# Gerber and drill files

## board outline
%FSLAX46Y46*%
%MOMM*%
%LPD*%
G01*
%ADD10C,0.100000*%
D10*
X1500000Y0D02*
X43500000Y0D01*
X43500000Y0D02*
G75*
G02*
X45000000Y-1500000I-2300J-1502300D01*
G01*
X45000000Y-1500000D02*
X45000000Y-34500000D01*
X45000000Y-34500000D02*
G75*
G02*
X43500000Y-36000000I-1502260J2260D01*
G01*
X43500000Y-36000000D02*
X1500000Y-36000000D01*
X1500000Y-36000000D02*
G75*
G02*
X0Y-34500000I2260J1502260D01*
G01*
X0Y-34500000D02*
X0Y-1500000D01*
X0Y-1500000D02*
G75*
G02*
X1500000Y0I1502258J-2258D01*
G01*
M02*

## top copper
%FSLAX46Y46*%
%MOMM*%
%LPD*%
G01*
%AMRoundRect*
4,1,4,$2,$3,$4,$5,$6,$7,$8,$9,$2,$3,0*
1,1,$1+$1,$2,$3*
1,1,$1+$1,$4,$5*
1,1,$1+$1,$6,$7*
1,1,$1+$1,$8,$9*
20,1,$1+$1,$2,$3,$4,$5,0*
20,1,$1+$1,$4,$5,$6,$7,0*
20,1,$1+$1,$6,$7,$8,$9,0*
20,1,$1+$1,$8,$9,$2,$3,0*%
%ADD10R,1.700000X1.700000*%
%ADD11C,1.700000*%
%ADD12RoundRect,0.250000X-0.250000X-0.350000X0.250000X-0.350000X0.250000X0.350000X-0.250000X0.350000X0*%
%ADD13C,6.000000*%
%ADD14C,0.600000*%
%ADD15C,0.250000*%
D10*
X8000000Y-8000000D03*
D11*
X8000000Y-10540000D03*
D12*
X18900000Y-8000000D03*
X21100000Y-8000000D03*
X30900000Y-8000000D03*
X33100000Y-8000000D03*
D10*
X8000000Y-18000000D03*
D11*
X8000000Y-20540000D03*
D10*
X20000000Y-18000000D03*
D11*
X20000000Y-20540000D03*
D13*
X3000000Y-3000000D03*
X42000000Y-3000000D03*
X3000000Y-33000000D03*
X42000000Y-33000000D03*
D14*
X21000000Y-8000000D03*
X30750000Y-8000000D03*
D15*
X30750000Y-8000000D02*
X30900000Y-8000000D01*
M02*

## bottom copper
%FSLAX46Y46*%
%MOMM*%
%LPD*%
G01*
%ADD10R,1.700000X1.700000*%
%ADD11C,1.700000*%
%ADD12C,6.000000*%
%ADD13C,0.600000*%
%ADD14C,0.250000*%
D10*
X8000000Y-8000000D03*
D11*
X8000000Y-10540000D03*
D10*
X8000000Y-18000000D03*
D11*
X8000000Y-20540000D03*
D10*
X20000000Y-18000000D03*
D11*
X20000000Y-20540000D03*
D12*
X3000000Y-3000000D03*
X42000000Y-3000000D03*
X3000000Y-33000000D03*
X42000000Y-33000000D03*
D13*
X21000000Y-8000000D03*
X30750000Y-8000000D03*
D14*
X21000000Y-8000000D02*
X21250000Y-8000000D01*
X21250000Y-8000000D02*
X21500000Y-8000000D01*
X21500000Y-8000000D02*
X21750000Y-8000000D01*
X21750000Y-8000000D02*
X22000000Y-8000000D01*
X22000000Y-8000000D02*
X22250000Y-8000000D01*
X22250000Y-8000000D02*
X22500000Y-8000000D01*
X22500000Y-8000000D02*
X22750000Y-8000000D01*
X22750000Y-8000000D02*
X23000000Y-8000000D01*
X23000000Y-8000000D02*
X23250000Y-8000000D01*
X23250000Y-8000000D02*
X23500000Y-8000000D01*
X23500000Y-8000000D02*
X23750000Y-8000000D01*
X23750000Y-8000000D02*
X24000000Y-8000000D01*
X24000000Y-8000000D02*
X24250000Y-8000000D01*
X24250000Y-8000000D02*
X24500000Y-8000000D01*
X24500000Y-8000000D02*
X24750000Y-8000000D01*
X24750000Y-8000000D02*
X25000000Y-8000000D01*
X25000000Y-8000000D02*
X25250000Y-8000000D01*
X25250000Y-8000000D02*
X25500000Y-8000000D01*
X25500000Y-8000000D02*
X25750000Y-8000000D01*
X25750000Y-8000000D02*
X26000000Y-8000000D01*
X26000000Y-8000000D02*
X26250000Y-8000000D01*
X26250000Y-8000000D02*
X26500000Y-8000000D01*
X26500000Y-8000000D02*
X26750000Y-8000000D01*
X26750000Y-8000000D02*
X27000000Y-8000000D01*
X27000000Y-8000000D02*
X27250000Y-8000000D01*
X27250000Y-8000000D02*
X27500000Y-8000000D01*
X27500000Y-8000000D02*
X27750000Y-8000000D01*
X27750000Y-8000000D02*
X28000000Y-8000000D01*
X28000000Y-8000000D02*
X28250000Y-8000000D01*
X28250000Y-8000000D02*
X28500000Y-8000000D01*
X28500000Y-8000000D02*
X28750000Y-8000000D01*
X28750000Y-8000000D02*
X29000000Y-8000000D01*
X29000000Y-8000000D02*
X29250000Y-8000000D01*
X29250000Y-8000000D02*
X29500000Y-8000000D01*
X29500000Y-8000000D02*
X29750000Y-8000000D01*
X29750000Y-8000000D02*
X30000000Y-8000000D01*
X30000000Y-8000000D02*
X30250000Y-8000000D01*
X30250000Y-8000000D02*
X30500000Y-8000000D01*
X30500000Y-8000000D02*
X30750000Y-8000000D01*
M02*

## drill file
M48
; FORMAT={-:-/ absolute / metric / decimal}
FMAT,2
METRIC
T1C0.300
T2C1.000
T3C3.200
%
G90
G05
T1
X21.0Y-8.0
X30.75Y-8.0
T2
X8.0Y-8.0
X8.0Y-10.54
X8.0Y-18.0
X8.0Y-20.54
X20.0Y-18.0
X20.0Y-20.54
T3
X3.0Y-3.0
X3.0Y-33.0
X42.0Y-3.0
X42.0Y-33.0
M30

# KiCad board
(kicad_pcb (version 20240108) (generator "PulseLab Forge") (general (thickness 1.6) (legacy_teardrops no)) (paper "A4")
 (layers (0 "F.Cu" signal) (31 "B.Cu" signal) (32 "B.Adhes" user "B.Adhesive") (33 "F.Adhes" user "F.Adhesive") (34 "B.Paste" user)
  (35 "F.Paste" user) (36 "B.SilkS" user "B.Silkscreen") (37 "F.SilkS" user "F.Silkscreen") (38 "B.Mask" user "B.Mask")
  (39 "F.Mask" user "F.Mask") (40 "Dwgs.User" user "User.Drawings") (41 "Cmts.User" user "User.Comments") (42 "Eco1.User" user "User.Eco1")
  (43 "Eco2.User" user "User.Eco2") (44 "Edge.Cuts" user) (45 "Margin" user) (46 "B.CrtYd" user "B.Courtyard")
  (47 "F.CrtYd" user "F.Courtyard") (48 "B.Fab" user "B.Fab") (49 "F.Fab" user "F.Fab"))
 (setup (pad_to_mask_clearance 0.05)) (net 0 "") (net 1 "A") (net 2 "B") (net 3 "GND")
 (gr_line (start 1.500 0.000) (end 43.500 0.000) (layer "Edge.Cuts") (stroke (width 0.1)))
 (gr_arc (start 43.500 0.000) (mid 44.560 0.440) (end 45.000 1.500) (layer "Edge.Cuts") (stroke (width 0.1)))
 (gr_line (start 45.000 1.500) (end 45.000 34.500) (layer "Edge.Cuts") (stroke (width 0.1)))
 (gr_arc (start 45.000 34.500) (mid 44.560 35.560) (end 43.500 36.000) (layer "Edge.Cuts") (stroke (width 0.1)))
 (gr_line (start 43.500 36.000) (end 1.500 36.000) (layer "Edge.Cuts") (stroke (width 0.1)))
 (gr_arc (start 1.500 36.000) (mid 0.440 35.560) (end 0.000 34.500) (layer "Edge.Cuts") (stroke (width 0.1)))
 (gr_line (start 0.000 34.500) (end 0.000 1.500) (layer "Edge.Cuts") (stroke (width 0.1)))
 (gr_arc (start 0.000 1.500) (mid 0.440 0.440) (end 1.500 0.000) (layer "Edge.Cuts") (stroke (width 0.1)))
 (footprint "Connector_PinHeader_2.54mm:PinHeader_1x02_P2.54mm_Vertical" (layer "F.Cu") (at 8.0000 8.0000)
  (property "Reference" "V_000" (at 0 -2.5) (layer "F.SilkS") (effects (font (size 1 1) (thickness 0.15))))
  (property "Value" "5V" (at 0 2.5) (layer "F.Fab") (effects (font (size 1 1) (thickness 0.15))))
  (pad "1" thru_hole rect (at 0.0000 0.0000) (size 1.7000 1.7000) (drill 1.0) (layers "*.Cu" "*.Mask") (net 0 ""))
  (pad "2" thru_hole circle (at 0.0000 2.5400) (size 1.7000 1.7000) (drill 1.0) (layers "*.Cu" "*.Mask") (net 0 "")))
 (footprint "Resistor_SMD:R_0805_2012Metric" (layer "F.Cu") (at 20.0000 8.0000)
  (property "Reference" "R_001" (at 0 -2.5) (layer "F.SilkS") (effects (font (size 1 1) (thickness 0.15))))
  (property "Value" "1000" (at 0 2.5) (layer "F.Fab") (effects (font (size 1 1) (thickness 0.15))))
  (pad "1" smd roundrect (at -1.1000 0.0000) (size 1.0000 1.2000) (layers "F.Cu" "F.Paste" "F.Mask") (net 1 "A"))
  (pad "2" smd roundrect (at 1.1000 0.0000) (size 1.0000 1.2000) (layers "F.Cu" "F.Paste" "F.Mask") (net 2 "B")))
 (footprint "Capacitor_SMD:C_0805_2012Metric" (layer "F.Cu") (at 32.0000 8.0000)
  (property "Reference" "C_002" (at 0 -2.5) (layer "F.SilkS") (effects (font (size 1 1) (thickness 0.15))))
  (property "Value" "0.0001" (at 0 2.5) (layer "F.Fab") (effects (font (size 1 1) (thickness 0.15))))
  (pad "1" smd roundrect (at -1.1000 0.0000) (size 1.0000 1.2000) (layers "F.Cu" "F.Paste" "F.Mask") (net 2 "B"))
  (pad "2" smd roundrect (at 1.1000 0.0000) (size 1.0000 1.2000) (layers "F.Cu" "F.Paste" "F.Mask") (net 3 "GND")))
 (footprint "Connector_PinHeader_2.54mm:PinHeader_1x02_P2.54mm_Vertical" (layer "F.Cu") (at 8.0000 18.0000)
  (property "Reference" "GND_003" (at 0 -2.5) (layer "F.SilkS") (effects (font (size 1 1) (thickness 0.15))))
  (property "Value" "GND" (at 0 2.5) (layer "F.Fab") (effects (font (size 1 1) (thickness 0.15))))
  (pad "1" thru_hole rect (at 0.0000 0.0000) (size 1.7000 1.7000) (drill 1.0) (layers "*.Cu" "*.Mask") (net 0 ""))
  (pad "2" thru_hole circle (at 0.0000 2.5400) (size 1.7000 1.7000) (drill 1.0) (layers "*.Cu" "*.Mask") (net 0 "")))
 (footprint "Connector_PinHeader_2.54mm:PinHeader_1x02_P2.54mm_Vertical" (layer "F.Cu") (at 20.0000 18.0000)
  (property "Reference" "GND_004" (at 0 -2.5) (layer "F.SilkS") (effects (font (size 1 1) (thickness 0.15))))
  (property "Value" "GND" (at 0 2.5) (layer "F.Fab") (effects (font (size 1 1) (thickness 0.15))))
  (pad "1" thru_hole rect (at 0.0000 0.0000) (size 1.7000 1.7000) (drill 1.0) (layers "*.Cu" "*.Mask") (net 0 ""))
  (pad "2" thru_hole circle (at 0.0000 2.5400) (size 1.7000 1.7000) (drill 1.0) (layers "*.Cu" "*.Mask") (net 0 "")))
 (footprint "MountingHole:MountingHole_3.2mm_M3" (layer "F.Cu") (at 3.0000 3.0000)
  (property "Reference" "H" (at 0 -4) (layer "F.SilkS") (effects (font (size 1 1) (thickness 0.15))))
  (pad "" thru_hole circle (at 0 0) (size 6.00 6.00) (drill 3.20) (layers "*.Cu" "*.Mask")))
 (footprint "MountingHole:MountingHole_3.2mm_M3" (layer "F.Cu") (at 42.0000 3.0000)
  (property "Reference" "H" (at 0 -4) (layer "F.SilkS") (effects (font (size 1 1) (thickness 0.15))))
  (pad "" thru_hole circle (at 0 0) (size 6.00 6.00) (drill 3.20) (layers "*.Cu" "*.Mask")))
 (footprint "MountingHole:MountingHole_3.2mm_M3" (layer "F.Cu") (at 3.0000 33.0000)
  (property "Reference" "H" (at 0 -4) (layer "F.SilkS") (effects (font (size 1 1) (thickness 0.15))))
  (pad "" thru_hole circle (at 0 0) (size 6.00 6.00) (drill 3.20) (layers "*.Cu" "*.Mask")))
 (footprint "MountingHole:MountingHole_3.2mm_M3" (layer "F.Cu") (at 42.0000 33.0000)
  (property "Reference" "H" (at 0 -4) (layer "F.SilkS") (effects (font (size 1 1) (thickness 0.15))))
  (pad "" thru_hole circle (at 0 0) (size 6.00 6.00) (drill 3.20) (layers "*.Cu" "*.Mask")))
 (segment (start 21.0000 8.0000) (end 21.2500 8.0000) (width 0.2500) (layer "B.Cu") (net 2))
 (segment (start 21.2500 8.0000) (end 21.5000 8.0000) (width 0.2500) (layer "B.Cu") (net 2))
 (segment (start 21.5000 8.0000) (end 21.7500 8.0000) (width 0.2500) (layer "B.Cu") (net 2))
 (segment (start 21.7500 8.0000) (end 22.0000 8.0000) (width 0.2500) (layer "B.Cu") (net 2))
 (segment (start 22.0000 8.0000) (end 22.2500 8.0000) (width 0.2500) (layer "B.Cu") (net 2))
 (segment (start 22.2500 8.0000) (end 22.5000 8.0000) (width 0.2500) (layer "B.Cu") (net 2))
 (segment (start 22.5000 8.0000) (end 22.7500 8.0000) (width 0.2500) (layer "B.Cu") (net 2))
 (segment (start 22.7500 8.0000) (end 23.0000 8.0000) (width 0.2500) (layer "B.Cu") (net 2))
 (segment (start 23.0000 8.0000) (end 23.2500 8.0000) (width 0.2500) (layer "B.Cu") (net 2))
 (segment (start 23.2500 8.0000) (end 23.5000 8.0000) (width 0.2500) (layer "B.Cu") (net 2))
 (segment (start 23.5000 8.0000) (end 23.7500 8.0000) (width 0.2500) (layer "B.Cu") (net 2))
 (segment (start 23.7500 8.0000) (end 24.0000 8.0000) (width 0.2500) (layer "B.Cu") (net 2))
 (segment (start 24.0000 8.0000) (end 24.2500 8.0000) (width 0.2500) (layer "B.Cu") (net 2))
 (segment (start 24.2500 8.0000) (end 24.5000 8.0000) (width 0.2500) (layer "B.Cu") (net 2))
 (segment (start 24.5000 8.0000) (end 24.7500 8.0000) (width 0.2500) (layer "B.Cu") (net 2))
 (segment (start 24.7500 8.0000) (end 25.0000 8.0000) (width 0.2500) (layer "B.Cu") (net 2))
 (segment (start 25.0000 8.0000) (end 25.2500 8.0000) (width 0.2500) (layer "B.Cu") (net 2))
 (segment (start 25.2500 8.0000) (end 25.5000 8.0000) (width 0.2500) (layer "B.Cu") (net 2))
 (segment (start 25.5000 8.0000) (end 25.7500 8.0000) (width 0.2500) (layer "B.Cu") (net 2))
 (segment (start 25.7500 8.0000) (end 26.0000 8.0000) (width 0.2500) (layer "B.Cu") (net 2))
 (segment (start 26.0000 8.0000) (end 26.2500 8.0000) (width 0.2500) (layer "B.Cu") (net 2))
 (segment (start 26.2500 8.0000) (end 26.5000 8.0000) (width 0.2500) (layer "B.Cu") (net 2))
 (segment (start 26.5000 8.0000) (end 26.7500 8.0000) (width 0.2500) (layer "B.Cu") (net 2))
 (segment (start 26.7500 8.0000) (end 27.0000 8.0000) (width 0.2500) (layer "B.Cu") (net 2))
 (segment (start 27.0000 8.0000) (end 27.2500 8.0000) (width 0.2500) (layer "B.Cu") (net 2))
 (segment (start 27.2500 8.0000) (end 27.5000 8.0000) (width 0.2500) (layer "B.Cu") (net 2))
 (segment (start 27.5000 8.0000) (end 27.7500 8.0000) (width 0.2500) (layer "B.Cu") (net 2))
 (segment (start 27.7500 8.0000) (end 28.0000 8.0000) (width 0.2500) (layer "B.Cu") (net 2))
 (segment (start 28.0000 8.0000) (end 28.2500 8.0000) (width 0.2500) (layer "B.Cu") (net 2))
 (segment (start 28.2500 8.0000) (end 28.5000 8.0000) (width 0.2500) (layer "B.Cu") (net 2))
 (segment (start 28.5000 8.0000) (end 28.7500 8.0000) (width 0.2500) (layer "B.Cu") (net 2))
 (segment (start 28.7500 8.0000) (end 29.0000 8.0000) (width 0.2500) (layer "B.Cu") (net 2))
 (segment (start 29.0000 8.0000) (end 29.2500 8.0000) (width 0.2500) (layer "B.Cu") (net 2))
 (segment (start 29.2500 8.0000) (end 29.5000 8.0000) (width 0.2500) (layer "B.Cu") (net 2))
 (segment (start 29.5000 8.0000) (end 29.7500 8.0000) (width 0.2500) (layer "B.Cu") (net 2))
 (segment (start 29.7500 8.0000) (end 30.0000 8.0000) (width 0.2500) (layer "B.Cu") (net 2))
 (segment (start 30.0000 8.0000) (end 30.2500 8.0000) (width 0.2500) (layer "B.Cu") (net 2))
 (segment (start 30.2500 8.0000) (end 30.5000 8.0000) (width 0.2500) (layer "B.Cu") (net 2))
 (segment (start 30.5000 8.0000) (end 30.7500 8.0000) (width 0.2500) (layer "B.Cu") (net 2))
 (segment (start 30.7500 8.0000) (end 30.9000 8.0000) (width 0.2500) (layer "F.Cu") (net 2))
 (via (at 21.0000 8.0000) (size 0.6000) (drill 0.3000) (layers "F.Cu" "B.Cu") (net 2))
 (via (at 30.7500 8.0000) (size 0.6000) (drill 0.3000) (layers "F.Cu" "B.Cu") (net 2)))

